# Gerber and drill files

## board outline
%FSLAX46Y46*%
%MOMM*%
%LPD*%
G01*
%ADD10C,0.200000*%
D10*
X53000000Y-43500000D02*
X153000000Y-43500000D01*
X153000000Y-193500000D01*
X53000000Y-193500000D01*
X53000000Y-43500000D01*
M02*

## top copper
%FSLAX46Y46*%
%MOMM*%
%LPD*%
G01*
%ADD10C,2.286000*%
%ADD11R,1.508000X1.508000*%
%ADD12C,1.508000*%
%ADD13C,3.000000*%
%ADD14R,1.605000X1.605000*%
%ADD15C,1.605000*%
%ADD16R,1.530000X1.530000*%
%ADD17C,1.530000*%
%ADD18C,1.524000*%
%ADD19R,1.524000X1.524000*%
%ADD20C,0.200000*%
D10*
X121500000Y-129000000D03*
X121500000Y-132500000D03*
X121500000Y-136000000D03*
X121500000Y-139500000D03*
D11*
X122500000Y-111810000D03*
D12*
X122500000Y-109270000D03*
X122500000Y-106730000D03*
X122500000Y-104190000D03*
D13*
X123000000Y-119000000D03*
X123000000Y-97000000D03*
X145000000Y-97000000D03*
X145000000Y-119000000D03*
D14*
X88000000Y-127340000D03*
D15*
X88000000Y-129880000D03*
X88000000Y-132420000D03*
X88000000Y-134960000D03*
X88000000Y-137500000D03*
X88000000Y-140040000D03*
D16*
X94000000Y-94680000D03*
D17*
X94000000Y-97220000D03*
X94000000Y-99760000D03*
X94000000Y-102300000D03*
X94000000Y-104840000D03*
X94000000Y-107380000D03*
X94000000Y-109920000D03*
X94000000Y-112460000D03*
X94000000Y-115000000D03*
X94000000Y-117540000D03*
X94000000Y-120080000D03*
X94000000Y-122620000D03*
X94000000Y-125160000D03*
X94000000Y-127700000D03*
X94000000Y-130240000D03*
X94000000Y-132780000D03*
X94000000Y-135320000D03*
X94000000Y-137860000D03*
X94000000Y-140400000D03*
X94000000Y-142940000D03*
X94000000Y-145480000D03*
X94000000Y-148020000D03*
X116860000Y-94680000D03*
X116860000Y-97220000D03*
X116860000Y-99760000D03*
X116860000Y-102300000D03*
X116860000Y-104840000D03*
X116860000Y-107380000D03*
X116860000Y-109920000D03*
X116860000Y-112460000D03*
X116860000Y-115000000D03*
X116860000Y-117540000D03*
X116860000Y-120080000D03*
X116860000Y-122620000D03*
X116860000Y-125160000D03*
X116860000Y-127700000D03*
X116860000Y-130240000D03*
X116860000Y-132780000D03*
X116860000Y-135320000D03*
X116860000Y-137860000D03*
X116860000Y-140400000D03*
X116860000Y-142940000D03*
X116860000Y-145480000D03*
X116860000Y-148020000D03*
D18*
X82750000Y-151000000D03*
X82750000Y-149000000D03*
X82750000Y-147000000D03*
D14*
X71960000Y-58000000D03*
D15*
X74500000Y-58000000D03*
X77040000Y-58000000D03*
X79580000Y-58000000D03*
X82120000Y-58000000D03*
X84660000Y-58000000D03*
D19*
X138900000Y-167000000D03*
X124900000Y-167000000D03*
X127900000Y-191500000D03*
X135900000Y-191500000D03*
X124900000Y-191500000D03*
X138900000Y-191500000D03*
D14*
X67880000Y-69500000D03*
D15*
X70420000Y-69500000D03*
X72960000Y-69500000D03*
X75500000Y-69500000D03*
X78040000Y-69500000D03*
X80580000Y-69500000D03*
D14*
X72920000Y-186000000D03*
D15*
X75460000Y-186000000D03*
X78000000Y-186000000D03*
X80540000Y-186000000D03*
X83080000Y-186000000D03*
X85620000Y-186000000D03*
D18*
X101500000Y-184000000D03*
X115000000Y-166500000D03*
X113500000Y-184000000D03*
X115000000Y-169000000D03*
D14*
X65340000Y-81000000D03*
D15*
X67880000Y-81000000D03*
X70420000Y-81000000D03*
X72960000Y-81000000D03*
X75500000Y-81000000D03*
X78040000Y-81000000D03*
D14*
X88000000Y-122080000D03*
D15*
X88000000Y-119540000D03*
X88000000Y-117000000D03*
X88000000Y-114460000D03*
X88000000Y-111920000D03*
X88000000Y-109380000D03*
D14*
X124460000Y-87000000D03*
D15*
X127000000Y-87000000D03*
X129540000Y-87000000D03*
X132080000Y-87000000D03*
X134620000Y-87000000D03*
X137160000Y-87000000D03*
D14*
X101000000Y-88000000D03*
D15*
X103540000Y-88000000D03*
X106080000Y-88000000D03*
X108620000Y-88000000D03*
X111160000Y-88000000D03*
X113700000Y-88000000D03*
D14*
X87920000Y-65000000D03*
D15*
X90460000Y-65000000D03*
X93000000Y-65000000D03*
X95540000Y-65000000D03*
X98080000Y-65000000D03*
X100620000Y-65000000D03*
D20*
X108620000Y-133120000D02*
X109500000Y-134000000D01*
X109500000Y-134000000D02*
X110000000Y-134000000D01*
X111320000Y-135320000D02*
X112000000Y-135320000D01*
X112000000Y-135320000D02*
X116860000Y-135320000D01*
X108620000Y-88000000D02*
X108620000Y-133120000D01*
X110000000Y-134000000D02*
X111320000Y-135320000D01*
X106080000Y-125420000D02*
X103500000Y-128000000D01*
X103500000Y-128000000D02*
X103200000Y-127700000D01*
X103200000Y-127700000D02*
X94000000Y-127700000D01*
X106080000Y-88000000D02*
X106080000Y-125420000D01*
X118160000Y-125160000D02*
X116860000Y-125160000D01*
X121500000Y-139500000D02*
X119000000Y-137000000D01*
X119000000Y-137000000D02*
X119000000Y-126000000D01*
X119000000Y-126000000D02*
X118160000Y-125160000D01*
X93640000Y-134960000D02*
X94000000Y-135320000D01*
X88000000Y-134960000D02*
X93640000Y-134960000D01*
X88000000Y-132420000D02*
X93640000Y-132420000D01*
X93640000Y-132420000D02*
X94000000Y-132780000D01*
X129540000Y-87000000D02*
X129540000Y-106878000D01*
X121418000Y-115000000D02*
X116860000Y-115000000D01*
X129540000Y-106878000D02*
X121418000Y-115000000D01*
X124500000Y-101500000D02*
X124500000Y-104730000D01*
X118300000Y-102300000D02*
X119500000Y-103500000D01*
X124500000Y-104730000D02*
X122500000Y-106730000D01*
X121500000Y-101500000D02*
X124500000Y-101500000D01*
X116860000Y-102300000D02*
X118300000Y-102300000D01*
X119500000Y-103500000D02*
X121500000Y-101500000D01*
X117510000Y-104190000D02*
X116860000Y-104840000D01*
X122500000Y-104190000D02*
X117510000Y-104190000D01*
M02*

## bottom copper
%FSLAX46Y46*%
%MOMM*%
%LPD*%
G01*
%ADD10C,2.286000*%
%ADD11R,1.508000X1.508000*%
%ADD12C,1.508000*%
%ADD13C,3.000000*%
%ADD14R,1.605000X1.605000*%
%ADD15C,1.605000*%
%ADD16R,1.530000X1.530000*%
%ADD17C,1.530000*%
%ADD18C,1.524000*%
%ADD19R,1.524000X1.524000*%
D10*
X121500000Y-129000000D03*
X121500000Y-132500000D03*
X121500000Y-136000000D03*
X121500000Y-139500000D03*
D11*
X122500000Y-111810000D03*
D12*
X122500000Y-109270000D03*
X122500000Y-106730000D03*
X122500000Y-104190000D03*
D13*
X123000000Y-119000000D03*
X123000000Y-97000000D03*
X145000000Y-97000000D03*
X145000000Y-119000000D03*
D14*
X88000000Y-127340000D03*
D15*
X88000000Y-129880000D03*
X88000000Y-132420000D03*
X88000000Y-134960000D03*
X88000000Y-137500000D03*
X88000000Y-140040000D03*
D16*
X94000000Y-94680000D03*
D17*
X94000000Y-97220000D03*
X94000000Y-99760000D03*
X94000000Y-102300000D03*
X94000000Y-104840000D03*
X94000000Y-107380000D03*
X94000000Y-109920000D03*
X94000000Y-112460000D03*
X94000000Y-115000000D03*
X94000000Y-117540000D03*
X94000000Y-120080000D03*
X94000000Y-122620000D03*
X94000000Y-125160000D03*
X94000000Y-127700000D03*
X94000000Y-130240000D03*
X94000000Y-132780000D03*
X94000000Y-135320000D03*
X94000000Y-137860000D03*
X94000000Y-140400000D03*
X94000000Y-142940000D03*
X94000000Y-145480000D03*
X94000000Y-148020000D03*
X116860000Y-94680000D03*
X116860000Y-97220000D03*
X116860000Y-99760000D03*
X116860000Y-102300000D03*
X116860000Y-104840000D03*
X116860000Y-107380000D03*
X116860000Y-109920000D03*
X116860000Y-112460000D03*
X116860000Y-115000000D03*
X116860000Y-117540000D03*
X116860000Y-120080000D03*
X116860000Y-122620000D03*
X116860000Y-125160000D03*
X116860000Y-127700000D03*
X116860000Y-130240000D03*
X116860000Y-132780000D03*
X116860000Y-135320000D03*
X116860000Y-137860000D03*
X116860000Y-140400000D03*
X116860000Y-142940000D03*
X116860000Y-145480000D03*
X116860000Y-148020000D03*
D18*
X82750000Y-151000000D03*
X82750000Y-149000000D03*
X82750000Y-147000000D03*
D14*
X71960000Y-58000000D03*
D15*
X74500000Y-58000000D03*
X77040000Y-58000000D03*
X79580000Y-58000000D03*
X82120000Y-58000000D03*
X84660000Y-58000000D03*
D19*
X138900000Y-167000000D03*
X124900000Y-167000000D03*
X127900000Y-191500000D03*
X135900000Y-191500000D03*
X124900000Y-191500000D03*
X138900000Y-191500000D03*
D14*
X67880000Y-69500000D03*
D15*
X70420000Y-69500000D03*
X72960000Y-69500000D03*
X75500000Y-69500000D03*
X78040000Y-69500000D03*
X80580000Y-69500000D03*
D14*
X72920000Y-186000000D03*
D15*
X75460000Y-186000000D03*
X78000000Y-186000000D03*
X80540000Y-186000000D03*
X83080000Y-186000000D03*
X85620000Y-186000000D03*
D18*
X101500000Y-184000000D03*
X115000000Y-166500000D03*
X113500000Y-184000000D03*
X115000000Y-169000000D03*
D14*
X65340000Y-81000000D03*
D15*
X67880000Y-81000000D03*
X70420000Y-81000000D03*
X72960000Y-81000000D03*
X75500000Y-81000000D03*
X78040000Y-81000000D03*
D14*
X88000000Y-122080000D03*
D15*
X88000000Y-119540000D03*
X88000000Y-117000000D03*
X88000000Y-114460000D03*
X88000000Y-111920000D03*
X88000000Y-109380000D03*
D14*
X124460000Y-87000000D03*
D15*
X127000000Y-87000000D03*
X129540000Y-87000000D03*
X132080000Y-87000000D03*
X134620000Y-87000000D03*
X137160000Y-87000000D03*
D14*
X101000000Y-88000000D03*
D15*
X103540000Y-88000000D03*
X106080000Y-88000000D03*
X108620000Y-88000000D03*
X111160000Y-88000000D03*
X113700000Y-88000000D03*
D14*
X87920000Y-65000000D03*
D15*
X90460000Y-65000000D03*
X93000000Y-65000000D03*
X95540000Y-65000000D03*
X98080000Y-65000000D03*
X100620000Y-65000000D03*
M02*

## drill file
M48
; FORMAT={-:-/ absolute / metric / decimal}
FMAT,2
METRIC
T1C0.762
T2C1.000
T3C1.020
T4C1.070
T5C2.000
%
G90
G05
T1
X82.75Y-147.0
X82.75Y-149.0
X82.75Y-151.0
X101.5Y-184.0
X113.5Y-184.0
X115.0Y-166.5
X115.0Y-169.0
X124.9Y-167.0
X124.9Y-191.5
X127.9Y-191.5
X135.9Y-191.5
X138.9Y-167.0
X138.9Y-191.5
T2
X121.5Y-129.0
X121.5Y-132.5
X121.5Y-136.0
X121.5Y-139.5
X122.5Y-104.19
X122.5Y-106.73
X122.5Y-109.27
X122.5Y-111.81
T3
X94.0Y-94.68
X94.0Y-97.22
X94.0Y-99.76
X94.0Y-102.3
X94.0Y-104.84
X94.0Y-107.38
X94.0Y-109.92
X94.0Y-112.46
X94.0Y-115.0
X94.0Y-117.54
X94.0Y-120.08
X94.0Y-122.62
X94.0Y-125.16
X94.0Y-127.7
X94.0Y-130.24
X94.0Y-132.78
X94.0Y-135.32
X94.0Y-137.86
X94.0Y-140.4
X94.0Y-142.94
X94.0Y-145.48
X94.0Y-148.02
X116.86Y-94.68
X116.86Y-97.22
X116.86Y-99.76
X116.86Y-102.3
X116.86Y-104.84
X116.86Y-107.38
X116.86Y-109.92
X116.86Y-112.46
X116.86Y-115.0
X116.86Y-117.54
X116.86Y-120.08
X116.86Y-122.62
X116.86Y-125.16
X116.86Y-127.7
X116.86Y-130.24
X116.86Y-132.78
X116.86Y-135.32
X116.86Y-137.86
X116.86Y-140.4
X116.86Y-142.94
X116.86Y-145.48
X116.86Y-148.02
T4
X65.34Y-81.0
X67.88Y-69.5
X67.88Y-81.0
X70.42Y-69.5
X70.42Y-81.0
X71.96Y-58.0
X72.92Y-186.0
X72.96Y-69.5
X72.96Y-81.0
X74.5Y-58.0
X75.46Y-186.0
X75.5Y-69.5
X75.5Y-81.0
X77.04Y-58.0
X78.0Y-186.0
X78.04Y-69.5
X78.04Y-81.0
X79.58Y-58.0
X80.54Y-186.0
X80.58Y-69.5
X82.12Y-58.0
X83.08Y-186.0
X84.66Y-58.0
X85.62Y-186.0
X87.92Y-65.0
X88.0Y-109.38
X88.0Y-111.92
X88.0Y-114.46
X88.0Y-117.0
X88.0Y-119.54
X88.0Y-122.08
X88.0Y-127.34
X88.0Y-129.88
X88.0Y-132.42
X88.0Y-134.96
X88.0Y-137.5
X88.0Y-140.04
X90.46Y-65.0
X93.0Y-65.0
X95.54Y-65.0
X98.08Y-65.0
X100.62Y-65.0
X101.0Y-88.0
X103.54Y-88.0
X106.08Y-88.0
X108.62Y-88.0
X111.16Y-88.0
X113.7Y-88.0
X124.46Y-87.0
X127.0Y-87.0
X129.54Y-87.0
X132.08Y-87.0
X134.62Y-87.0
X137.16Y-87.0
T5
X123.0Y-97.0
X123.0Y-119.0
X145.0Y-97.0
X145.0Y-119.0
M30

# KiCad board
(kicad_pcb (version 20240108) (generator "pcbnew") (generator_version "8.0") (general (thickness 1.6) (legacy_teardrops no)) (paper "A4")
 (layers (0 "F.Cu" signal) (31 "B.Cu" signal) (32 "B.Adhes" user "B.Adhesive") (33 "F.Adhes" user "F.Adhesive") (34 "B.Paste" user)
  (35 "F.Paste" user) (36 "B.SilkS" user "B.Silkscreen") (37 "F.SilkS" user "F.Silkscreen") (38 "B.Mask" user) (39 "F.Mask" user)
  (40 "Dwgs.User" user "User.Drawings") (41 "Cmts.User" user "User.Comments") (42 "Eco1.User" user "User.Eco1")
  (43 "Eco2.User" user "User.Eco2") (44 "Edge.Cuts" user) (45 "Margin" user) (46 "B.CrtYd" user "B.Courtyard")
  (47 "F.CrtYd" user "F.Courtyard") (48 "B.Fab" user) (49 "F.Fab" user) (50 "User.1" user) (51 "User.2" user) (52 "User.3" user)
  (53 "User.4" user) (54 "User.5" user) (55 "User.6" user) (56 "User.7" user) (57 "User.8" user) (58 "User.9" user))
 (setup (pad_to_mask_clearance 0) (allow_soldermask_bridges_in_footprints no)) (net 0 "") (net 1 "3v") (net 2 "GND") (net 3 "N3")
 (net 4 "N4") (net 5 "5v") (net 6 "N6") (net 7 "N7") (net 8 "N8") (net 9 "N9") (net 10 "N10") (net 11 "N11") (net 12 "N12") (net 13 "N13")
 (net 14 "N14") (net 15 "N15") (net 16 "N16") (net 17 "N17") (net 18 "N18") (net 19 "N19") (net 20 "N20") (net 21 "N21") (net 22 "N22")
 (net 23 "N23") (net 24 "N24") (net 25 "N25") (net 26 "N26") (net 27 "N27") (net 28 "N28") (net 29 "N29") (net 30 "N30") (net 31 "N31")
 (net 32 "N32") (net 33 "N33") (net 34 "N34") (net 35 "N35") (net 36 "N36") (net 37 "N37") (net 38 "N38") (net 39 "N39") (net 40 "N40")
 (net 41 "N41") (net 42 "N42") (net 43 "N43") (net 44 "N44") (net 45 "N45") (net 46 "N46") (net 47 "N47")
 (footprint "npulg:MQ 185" (layer "F.Cu") (at 144 132.5 -90)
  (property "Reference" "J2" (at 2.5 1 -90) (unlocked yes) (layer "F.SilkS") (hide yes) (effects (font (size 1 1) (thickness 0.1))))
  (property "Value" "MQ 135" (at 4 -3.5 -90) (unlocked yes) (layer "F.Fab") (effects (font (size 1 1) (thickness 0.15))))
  (pad "1" thru_hole circle (at -3.5 22.5 270) (size 2.286 2.286) (drill 1) (layers "*.Cu" "*.Mask") (remove_unused_layers no) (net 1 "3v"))
  (pad "2" thru_hole circle (at 0 22.5 270) (size 2.286 2.286) (drill 1) (layers "*.Cu" "*.Mask") (remove_unused_layers no) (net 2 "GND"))
  (pad "3" thru_hole circle (at 3.5 22.5 270) (size 2.286 2.286) (drill 1) (layers "*.Cu" "*.Mask") (remove_unused_layers no) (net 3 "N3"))
  (pad "4" thru_hole circle (at 7 22.5 270) (size 2.286 2.286) (drill 1) (layers "*.Cu" "*.Mask") (remove_unused_layers no) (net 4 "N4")))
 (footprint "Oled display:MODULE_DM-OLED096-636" (layer "F.Cu") (at 134 108 90)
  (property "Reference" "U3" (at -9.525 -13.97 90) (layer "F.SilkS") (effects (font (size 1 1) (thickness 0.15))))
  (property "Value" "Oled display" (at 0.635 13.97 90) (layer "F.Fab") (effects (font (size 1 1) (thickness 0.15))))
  (pad "1" thru_hole rect (at -3.81 -11.5 90) (size 1.508 1.508) (drill 1) (layers "*.Cu" "*.Mask") (remove_unused_layers no) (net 2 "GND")
   (solder_mask_margin 0.102))
  (pad "2" thru_hole circle (at -1.27 -11.5 90) (size 1.508 1.508) (drill 1) (layers "*.Cu" "*.Mask") (remove_unused_layers no) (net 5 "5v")
   (solder_mask_margin 0.102))
  (pad "3" thru_hole circle (at 1.27 -11.5 90) (size 1.508 1.508) (drill 1) (layers "*.Cu" "*.Mask") (remove_unused_layers no) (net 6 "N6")
   (solder_mask_margin 0.102))
  (pad "4" thru_hole circle (at 3.81 -11.5 90) (size 1.508 1.508) (drill 1) (layers "*.Cu" "*.Mask") (remove_unused_layers no) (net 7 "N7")
   (solder_mask_margin 0.102))
  (pad "S1" thru_hole circle (at -11 -11 90) (size 3 3) (drill 2) (layers "*.Cu" "*.Mask") (remove_unused_layers no)
   (solder_mask_margin 0.102))
  (pad "S2" thru_hole circle (at 11 -11 90) (size 3 3) (drill 2) (layers "*.Cu" "*.Mask") (remove_unused_layers no)
   (solder_mask_margin 0.102))
  (pad "S3" thru_hole circle (at 11 11 90) (size 3 3) (drill 2) (layers "*.Cu" "*.Mask") (remove_unused_layers no)
   (solder_mask_margin 0.102))
  (pad "S4" thru_hole circle (at -11 11 90) (size 3 3) (drill 2) (layers "*.Cu" "*.Mask") (remove_unused_layers no)
   (solder_mask_margin 0.102)))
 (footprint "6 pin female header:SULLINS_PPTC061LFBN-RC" (layer "F.Cu") (at 88 133.69 -90)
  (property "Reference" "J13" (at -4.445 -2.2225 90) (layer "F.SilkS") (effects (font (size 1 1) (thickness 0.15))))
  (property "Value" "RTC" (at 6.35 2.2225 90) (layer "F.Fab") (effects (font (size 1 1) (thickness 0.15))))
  (pad "1" thru_hole rect (at -6.35 0 270) (size 1.605 1.605) (drill 1.07) (layers "*.Cu" "*.Mask") (remove_unused_layers no) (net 5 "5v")
   (solder_mask_margin 0.102))
  (pad "2" thru_hole circle (at -3.81 0 270) (size 1.605 1.605) (drill 1.07) (layers "*.Cu" "*.Mask") (remove_unused_layers no)
   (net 2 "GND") (solder_mask_margin 0.102))
  (pad "3" thru_hole circle (at -1.27 0 270) (size 1.605 1.605) (drill 1.07) (layers "*.Cu" "*.Mask") (remove_unused_layers no) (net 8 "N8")
   (solder_mask_margin 0.102))
  (pad "4" thru_hole circle (at 1.27 0 270) (size 1.605 1.605) (drill 1.07) (layers "*.Cu" "*.Mask") (remove_unused_layers no) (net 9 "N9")
   (solder_mask_margin 0.102))
  (pad "5" thru_hole circle (at 3.81 0 270) (size 1.605 1.605) (drill 1.07) (layers "*.Cu" "*.Mask") (remove_unused_layers no)
   (solder_mask_margin 0.102))
  (pad "6" thru_hole circle (at 6.35 0 270) (size 1.605 1.605) (drill 1.07) (layers "*.Cu" "*.Mask") (remove_unused_layers no)
   (solder_mask_margin 0.102)))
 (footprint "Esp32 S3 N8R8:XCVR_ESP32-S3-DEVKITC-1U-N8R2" (layer "F.Cu") (at 105.43 124.65)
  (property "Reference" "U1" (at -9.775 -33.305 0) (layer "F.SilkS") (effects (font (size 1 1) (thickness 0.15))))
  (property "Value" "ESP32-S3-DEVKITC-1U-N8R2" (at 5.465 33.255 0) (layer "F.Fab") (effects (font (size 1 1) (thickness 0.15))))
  (pad "J1_1" thru_hole rect (at -11.43 -29.97) (size 1.53 1.53) (drill 1.02) (layers "*.Cu" "*.Mask") (remove_unused_layers no)
   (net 1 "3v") (solder_mask_margin 0.102))
  (pad "J1_2" thru_hole circle (at -11.43 -27.43) (size 1.53 1.53) (drill 1.02) (layers "*.Cu" "*.Mask") (remove_unused_layers no)
   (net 1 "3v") (solder_mask_margin 0.102))
  (pad "J1_3" thru_hole circle (at -11.43 -24.89) (size 1.53 1.53) (drill 1.02) (layers "*.Cu" "*.Mask") (remove_unused_layers no)
   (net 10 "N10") (solder_mask_margin 0.102))
  (pad "J1_4" thru_hole circle (at -11.43 -22.35) (size 1.53 1.53) (drill 1.02) (layers "*.Cu" "*.Mask") (remove_unused_layers no)
   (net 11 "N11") (solder_mask_margin 0.102))
  (pad "J1_5" thru_hole circle (at -11.43 -19.81) (size 1.53 1.53) (drill 1.02) (layers "*.Cu" "*.Mask") (remove_unused_layers no)
   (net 5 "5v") (solder_mask_margin 0.102))
  (pad "J1_6" thru_hole circle (at -11.43 -17.27) (size 1.53 1.53) (drill 1.02) (layers "*.Cu" "*.Mask") (remove_unused_layers no)
   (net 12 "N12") (solder_mask_margin 0.102))
  (pad "J1_7" thru_hole circle (at -11.43 -14.73) (size 1.53 1.53) (drill 1.02) (layers "*.Cu" "*.Mask") (remove_unused_layers no)
   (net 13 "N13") (solder_mask_margin 0.102))
  (pad "J1_8" thru_hole circle (at -11.43 -12.19) (size 1.53 1.53) (drill 1.02) (layers "*.Cu" "*.Mask") (remove_unused_layers no)
   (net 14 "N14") (solder_mask_margin 0.102))
  (pad "J1_9" thru_hole circle (at -11.43 -9.65) (size 1.53 1.53) (drill 1.02) (layers "*.Cu" "*.Mask") (remove_unused_layers no)
   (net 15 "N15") (solder_mask_margin 0.102))
  (pad "J1_10" thru_hole circle (at -11.43 -7.11) (size 1.53 1.53) (drill 1.02) (layers "*.Cu" "*.Mask") (remove_unused_layers no)
   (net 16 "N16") (solder_mask_margin 0.102))
  (pad "J1_11" thru_hole circle (at -11.43 -4.57) (size 1.53 1.53) (drill 1.02) (layers "*.Cu" "*.Mask") (remove_unused_layers no)
   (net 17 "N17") (solder_mask_margin 0.102))
  (pad "J1_12" thru_hole circle (at -11.43 -2.03) (size 1.53 1.53) (drill 1.02) (layers "*.Cu" "*.Mask") (remove_unused_layers no)
   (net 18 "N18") (solder_mask_margin 0.102))
  (pad "J1_13" thru_hole circle (at -11.43 0.51) (size 1.53 1.53) (drill 1.02) (layers "*.Cu" "*.Mask") (remove_unused_layers no)
   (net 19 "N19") (solder_mask_margin 0.102))
  (pad "J1_14" thru_hole circle (at -11.43 3.05) (size 1.53 1.53) (drill 1.02) (layers "*.Cu" "*.Mask") (remove_unused_layers no)
   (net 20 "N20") (solder_mask_margin 0.102))
  (pad "J1_15" thru_hole circle (at -11.43 5.59) (size 1.53 1.53) (drill 1.02) (layers "*.Cu" "*.Mask") (remove_unused_layers no)
   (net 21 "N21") (solder_mask_margin 0.102))
  (pad "J1_16" thru_hole circle (at -11.43 8.13) (size 1.53 1.53) (drill 1.02) (layers "*.Cu" "*.Mask") (remove_unused_layers no)
   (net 8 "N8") (solder_mask_margin 0.102))
  (pad "J1_17" thru_hole circle (at -11.43 10.67) (size 1.53 1.53) (drill 1.02) (layers "*.Cu" "*.Mask") (remove_unused_layers no)
   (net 9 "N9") (solder_mask_margin 0.102))
  (pad "J1_18" thru_hole circle (at -11.43 13.21) (size 1.53 1.53) (drill 1.02) (layers "*.Cu" "*.Mask") (remove_unused_layers no)
   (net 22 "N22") (solder_mask_margin 0.102))
  (pad "J1_19" thru_hole circle (at -11.43 15.75) (size 1.53 1.53) (drill 1.02) (layers "*.Cu" "*.Mask") (remove_unused_layers no)
   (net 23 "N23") (solder_mask_margin 0.102))
  (pad "J1_20" thru_hole circle (at -11.43 18.29) (size 1.53 1.53) (drill 1.02) (layers "*.Cu" "*.Mask") (remove_unused_layers no)
   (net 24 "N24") (solder_mask_margin 0.102))
  (pad "J1_21" thru_hole circle (at -11.43 20.83) (size 1.53 1.53) (drill 1.02) (layers "*.Cu" "*.Mask") (remove_unused_layers no)
   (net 5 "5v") (solder_mask_margin 0.102))
  (pad "J1_22" thru_hole circle (at -11.43 23.37) (size 1.53 1.53) (drill 1.02) (layers "*.Cu" "*.Mask") (remove_unused_layers no)
   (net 2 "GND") (solder_mask_margin 0.102))
  (pad "J3_1" thru_hole circle (at 11.43 -29.97) (size 1.53 1.53) (drill 1.02) (layers "*.Cu" "*.Mask") (remove_unused_layers no)
   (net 2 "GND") (solder_mask_margin 0.102))
  (pad "J3_2" thru_hole circle (at 11.43 -27.43) (size 1.53 1.53) (drill 1.02) (layers "*.Cu" "*.Mask") (remove_unused_layers no)
   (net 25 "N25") (solder_mask_margin 0.102))
  (pad "J3_3" thru_hole circle (at 11.43 -24.89) (size 1.53 1.53) (drill 1.02) (layers "*.Cu" "*.Mask") (remove_unused_layers no)
   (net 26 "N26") (solder_mask_margin 0.102))
  (pad "J3_4" thru_hole circle (at 11.43 -22.35) (size 1.53 1.53) (drill 1.02) (layers "*.Cu" "*.Mask") (remove_unused_layers no)
   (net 6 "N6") (solder_mask_margin 0.102))
  (pad "J3_5" thru_hole circle (at 11.43 -19.81) (size 1.53 1.53) (drill 1.02) (layers "*.Cu" "*.Mask") (remove_unused_layers no)
   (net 7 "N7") (solder_mask_margin 0.102))
  (pad "J3_6" thru_hole circle (at 11.43 -17.27) (size 1.53 1.53) (drill 1.02) (layers "*.Cu" "*.Mask") (remove_unused_layers no)
   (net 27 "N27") (solder_mask_margin 0.102))
  (pad "J3_7" thru_hole circle (at 11.43 -14.73) (size 1.53 1.53) (drill 1.02) (layers "*.Cu" "*.Mask") (remove_unused_layers no)
   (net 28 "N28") (solder_mask_margin 0.102))
  (pad "J3_8" thru_hole circle (at 11.43 -12.19) (size 1.53 1.53) (drill 1.02) (layers "*.Cu" "*.Mask") (remove_unused_layers no)
   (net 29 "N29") (solder_mask_margin 0.102))
  (pad "J3_9" thru_hole circle (at 11.43 -9.65) (size 1.53 1.53) (drill 1.02) (layers "*.Cu" "*.Mask") (remove_unused_layers no)
   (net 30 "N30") (solder_mask_margin 0.102))
  (pad "J3_10" thru_hole circle (at 11.43 -7.11) (size 1.53 1.53) (drill 1.02) (layers "*.Cu" "*.Mask") (remove_unused_layers no)
   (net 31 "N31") (solder_mask_margin 0.102))
  (pad "J3_11" thru_hole circle (at 11.43 -4.57) (size 1.53 1.53) (drill 1.02) (layers "*.Cu" "*.Mask") (remove_unused_layers no)
   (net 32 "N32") (solder_mask_margin 0.102))
  (pad "J3_12" thru_hole circle (at 11.43 -2.03) (size 1.53 1.53) (drill 1.02) (layers "*.Cu" "*.Mask") (remove_unused_layers no)
   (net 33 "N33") (solder_mask_margin 0.102))
  (pad "J3_13" thru_hole circle (at 11.43 0.51) (size 1.53 1.53) (drill 1.02) (layers "*.Cu" "*.Mask") (remove_unused_layers no)
   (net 4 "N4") (solder_mask_margin 0.102))
  (pad "J3_14" thru_hole circle (at 11.43 3.05) (size 1.53 1.53) (drill 1.02) (layers "*.Cu" "*.Mask") (remove_unused_layers no)
   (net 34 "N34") (solder_mask_margin 0.102))
  (pad "J3_15" thru_hole circle (at 11.43 5.59) (size 1.53 1.53) (drill 1.02) (layers "*.Cu" "*.Mask") (remove_unused_layers no)
   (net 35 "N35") (solder_mask_margin 0.102))
  (pad "J3_16" thru_hole circle (at 11.43 8.13) (size 1.53 1.53) (drill 1.02) (layers "*.Cu" "*.Mask") (remove_unused_layers no)
   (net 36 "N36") (solder_mask_margin 0.102))
  (pad "J3_17" thru_hole circle (at 11.43 10.67) (size 1.53 1.53) (drill 1.02) (layers "*.Cu" "*.Mask") (remove_unused_layers no)
   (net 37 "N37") (solder_mask_margin 0.102))
  (pad "J3_18" thru_hole circle (at 11.43 13.21) (size 1.53 1.53) (drill 1.02) (layers "*.Cu" "*.Mask") (remove_unused_layers no)
   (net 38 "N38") (solder_mask_margin 0.102))
  (pad "J3_19" thru_hole circle (at 11.43 15.75) (size 1.53 1.53) (drill 1.02) (layers "*.Cu" "*.Mask") (remove_unused_layers no)
   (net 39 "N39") (solder_mask_margin 0.102))
  (pad "J3_20" thru_hole circle (at 11.43 18.29) (size 1.53 1.53) (drill 1.02) (layers "*.Cu" "*.Mask") (remove_unused_layers no)
   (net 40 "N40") (solder_mask_margin 0.102))
  (pad "J3_21" thru_hole circle (at 11.43 20.83) (size 1.53 1.53) (drill 1.02) (layers "*.Cu" "*.Mask") (remove_unused_layers no)
   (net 2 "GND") (solder_mask_margin 0.102))
  (pad "J3_22" thru_hole circle (at 11.43 23.37) (size 1.53 1.53) (drill 1.02) (layers "*.Cu" "*.Mask") (remove_unused_layers no)
   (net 2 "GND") (solder_mask_margin 0.102)))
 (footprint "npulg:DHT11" (layer "F.Cu") (at 75.25 148 90)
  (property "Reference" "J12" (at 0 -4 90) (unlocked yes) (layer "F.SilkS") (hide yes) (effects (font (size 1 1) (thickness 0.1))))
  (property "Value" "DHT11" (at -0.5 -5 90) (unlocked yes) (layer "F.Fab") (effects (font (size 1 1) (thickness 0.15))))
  (pad "1" thru_hole circle (at -3 7.5 90) (size 1.524 1.524) (drill 0.762) (layers "*.Cu" "*.Mask") (remove_unused_layers no) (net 2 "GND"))
  (pad "2" thru_hole circle (at -1 7.5 90) (size 1.524 1.524) (drill 0.762) (layers "*.Cu" "*.Mask") (remove_unused_layers no)
   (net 33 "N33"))
  (pad "3" thru_hole circle (at 1 7.5 90) (size 1.524 1.524) (drill 0.762) (layers "*.Cu" "*.Mask") (remove_unused_layers no) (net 5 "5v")))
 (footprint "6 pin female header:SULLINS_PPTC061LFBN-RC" (layer "F.Cu") (at 78.31 58)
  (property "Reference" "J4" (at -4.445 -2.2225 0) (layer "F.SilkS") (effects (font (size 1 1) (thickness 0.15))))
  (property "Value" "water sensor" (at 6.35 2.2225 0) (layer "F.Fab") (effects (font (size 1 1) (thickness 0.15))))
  (pad "1" thru_hole rect (at -6.35 0) (size 1.605 1.605) (drill 1.07) (layers "*.Cu" "*.Mask") (remove_unused_layers no) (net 5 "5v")
   (solder_mask_margin 0.102))
  (pad "2" thru_hole circle (at -3.81 0) (size 1.605 1.605) (drill 1.07) (layers "*.Cu" "*.Mask") (remove_unused_layers no) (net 2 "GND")
   (solder_mask_margin 0.102))
  (pad "3" thru_hole circle (at -1.27 0) (size 1.605 1.605) (drill 1.07) (layers "*.Cu" "*.Mask") (remove_unused_layers no) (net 11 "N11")
   (solder_mask_margin 0.102))
  (pad "4" thru_hole circle (at 1.27 0) (size 1.605 1.605) (drill 1.07) (layers "*.Cu" "*.Mask") (remove_unused_layers no)
   (solder_mask_margin 0.102))
  (pad "5" thru_hole circle (at 3.81 0) (size 1.605 1.605) (drill 1.07) (layers "*.Cu" "*.Mask") (remove_unused_layers no)
   (solder_mask_margin 0.102))
  (pad "6" thru_hole circle (at 6.35 0) (size 1.605 1.605) (drill 1.07) (layers "*.Cu" "*.Mask") (remove_unused_layers no)
   (solder_mask_margin 0.102)))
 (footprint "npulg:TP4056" (layer "F.Cu") (at 130.9 171.5)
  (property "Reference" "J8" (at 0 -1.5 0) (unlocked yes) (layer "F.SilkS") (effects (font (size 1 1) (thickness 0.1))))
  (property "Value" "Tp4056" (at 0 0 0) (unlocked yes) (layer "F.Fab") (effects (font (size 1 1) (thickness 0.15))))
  (pad "+IN" thru_hole rect (at 8 -4.5) (size 1.524 1.524) (drill 0.762) (layers "*.Cu" "*.Mask") (remove_unused_layers no))
  (pad "-IN" thru_hole rect (at -6 -4.5) (size 1.524 1.524) (drill 0.762) (layers "*.Cu" "*.Mask") (remove_unused_layers no))
  (pad "BAT+" thru_hole rect (at -3 20) (size 1.524 1.524) (drill 0.762) (layers "*.Cu" "*.Mask") (remove_unused_layers no))
  (pad "BAT-" thru_hole rect (at 5 20) (size 1.524 1.524) (drill 0.762) (layers "*.Cu" "*.Mask") (remove_unused_layers no))
  (pad "OUT+" thru_hole rect (at -6 20) (size 1.524 1.524) (drill 0.762) (layers "*.Cu" "*.Mask") (remove_unused_layers no))
  (pad "OUT-" thru_hole rect (at 8 20) (size 1.524 1.524) (drill 0.762) (layers "*.Cu" "*.Mask") (remove_unused_layers no)))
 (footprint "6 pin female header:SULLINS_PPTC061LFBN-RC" (layer "F.Cu") (at 74.23 69.5)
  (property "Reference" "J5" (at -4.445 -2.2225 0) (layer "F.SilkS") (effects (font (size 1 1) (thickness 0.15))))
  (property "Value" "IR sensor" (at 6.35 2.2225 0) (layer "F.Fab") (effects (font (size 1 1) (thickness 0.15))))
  (pad "1" thru_hole rect (at -6.35 0) (size 1.605 1.605) (drill 1.07) (layers "*.Cu" "*.Mask") (remove_unused_layers no) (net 5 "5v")
   (solder_mask_margin 0.102))
  (pad "2" thru_hole circle (at -3.81 0) (size 1.605 1.605) (drill 1.07) (layers "*.Cu" "*.Mask") (remove_unused_layers no) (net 2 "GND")
   (solder_mask_margin 0.102))
  (pad "3" thru_hole circle (at -1.27 0) (size 1.605 1.605) (drill 1.07) (layers "*.Cu" "*.Mask") (remove_unused_layers no) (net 36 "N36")
   (solder_mask_margin 0.102))
  (pad "4" thru_hole circle (at 1.27 0) (size 1.605 1.605) (drill 1.07) (layers "*.Cu" "*.Mask") (remove_unused_layers no)
   (solder_mask_margin 0.102))
  (pad "5" thru_hole circle (at 3.81 0) (size 1.605 1.605) (drill 1.07) (layers "*.Cu" "*.Mask") (remove_unused_layers no)
   (solder_mask_margin 0.102))
  (pad "6" thru_hole circle (at 6.35 0) (size 1.605 1.605) (drill 1.07) (layers "*.Cu" "*.Mask") (remove_unused_layers no)
   (solder_mask_margin 0.102)))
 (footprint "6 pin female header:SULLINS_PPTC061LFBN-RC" (layer "F.Cu") (at 79.27 186)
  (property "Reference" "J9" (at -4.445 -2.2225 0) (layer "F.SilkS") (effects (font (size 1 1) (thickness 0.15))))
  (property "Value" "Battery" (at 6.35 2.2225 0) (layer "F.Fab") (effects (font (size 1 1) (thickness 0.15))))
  (pad "1" thru_hole rect (at -6.35 0) (size 1.605 1.605) (drill 1.07) (layers "*.Cu" "*.Mask") (remove_unused_layers no) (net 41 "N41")
   (solder_mask_margin 0.102))
  (pad "2" thru_hole circle (at -3.81 0) (size 1.605 1.605) (drill 1.07) (layers "*.Cu" "*.Mask") (remove_unused_layers no) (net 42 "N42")
   (solder_mask_margin 0.102))
  (pad "3" thru_hole circle (at -1.27 0) (size 1.605 1.605) (drill 1.07) (layers "*.Cu" "*.Mask") (remove_unused_layers no)
   (solder_mask_margin 0.102))
  (pad "4" thru_hole circle (at 1.27 0) (size 1.605 1.605) (drill 1.07) (layers "*.Cu" "*.Mask") (remove_unused_layers no)
   (solder_mask_margin 0.102))
  (pad "5" thru_hole circle (at 3.81 0) (size 1.605 1.605) (drill 1.07) (layers "*.Cu" "*.Mask") (remove_unused_layers no)
   (solder_mask_margin 0.102))
  (pad "6" thru_hole circle (at 6.35 0) (size 1.605 1.605) (drill 1.07) (layers "*.Cu" "*.Mask") (remove_unused_layers no)
   (solder_mask_margin 0.102)))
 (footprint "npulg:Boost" (layer "F.Cu") (at 105.5 172)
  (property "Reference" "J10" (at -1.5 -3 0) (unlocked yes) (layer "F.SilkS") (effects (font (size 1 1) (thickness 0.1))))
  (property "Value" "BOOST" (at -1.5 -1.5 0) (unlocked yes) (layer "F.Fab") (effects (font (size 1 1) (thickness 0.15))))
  (pad "+" thru_hole circle (at -4 12) (size 1.524 1.524) (drill 0.762) (layers "*.Cu" "*.Mask") (remove_unused_layers no))
  (pad "+5v" thru_hole circle (at 9.5 -5.5) (size 1.524 1.524) (drill 0.762) (layers "*.Cu" "*.Mask") (remove_unused_layers no))
  (pad "-" thru_hole circle (at 8 12) (size 1.524 1.524) (drill 0.762) (layers "*.Cu" "*.Mask") (remove_unused_layers no))
  (pad "GND" thru_hole circle (at 9.5 -3) (size 1.524 1.524) (drill 0.762) (layers "*.Cu" "*.Mask") (remove_unused_layers no)))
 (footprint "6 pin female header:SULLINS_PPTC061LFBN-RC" (layer "F.Cu") (at 71.69 81)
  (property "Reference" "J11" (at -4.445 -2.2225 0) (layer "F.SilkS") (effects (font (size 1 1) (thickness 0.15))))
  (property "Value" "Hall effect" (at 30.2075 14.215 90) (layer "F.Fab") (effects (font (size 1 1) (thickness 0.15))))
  (pad "1" thru_hole rect (at -6.35 0) (size 1.605 1.605) (drill 1.07) (layers "*.Cu" "*.Mask") (remove_unused_layers no) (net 5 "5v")
   (solder_mask_margin 0.102))
  (pad "2" thru_hole circle (at -3.81 0) (size 1.605 1.605) (drill 1.07) (layers "*.Cu" "*.Mask") (remove_unused_layers no) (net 2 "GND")
   (solder_mask_margin 0.102))
  (pad "3" thru_hole circle (at -1.27 0) (size 1.605 1.605) (drill 1.07) (layers "*.Cu" "*.Mask") (remove_unused_layers no) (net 34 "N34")
   (solder_mask_margin 0.102))
  (pad "4" thru_hole circle (at 1.27 0) (size 1.605 1.605) (drill 1.07) (layers "*.Cu" "*.Mask") (remove_unused_layers no)
   (solder_mask_margin 0.102))
  (pad "5" thru_hole circle (at 3.81 0) (size 1.605 1.605) (drill 1.07) (layers "*.Cu" "*.Mask") (remove_unused_layers no)
   (solder_mask_margin 0.102))
  (pad "6" thru_hole circle (at 6.35 0) (size 1.605 1.605) (drill 1.07) (layers "*.Cu" "*.Mask") (remove_unused_layers no)
   (solder_mask_margin 0.102)))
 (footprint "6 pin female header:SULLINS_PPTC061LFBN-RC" (layer "F.Cu") (at 88 115.73 90)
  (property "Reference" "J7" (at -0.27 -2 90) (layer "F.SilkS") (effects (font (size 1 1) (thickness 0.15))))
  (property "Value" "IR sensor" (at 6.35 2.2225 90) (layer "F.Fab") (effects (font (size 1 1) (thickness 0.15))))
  (pad "1" thru_hole rect (at -6.35 0 90) (size 1.605 1.605) (drill 1.07) (layers "*.Cu" "*.Mask") (remove_unused_layers no) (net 5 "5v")
   (solder_mask_margin 0.102))
  (pad "2" thru_hole circle (at -3.81 0 90) (size 1.605 1.605) (drill 1.07) (layers "*.Cu" "*.Mask") (remove_unused_layers no) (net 2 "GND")
   (solder_mask_margin 0.102))
  (pad "3" thru_hole circle (at -1.27 0 90) (size 1.605 1.605) (drill 1.07) (layers "*.Cu" "*.Mask") (remove_unused_layers no)
   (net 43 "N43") (solder_mask_margin 0.102))
  (pad "4" thru_hole circle (at 1.27 0 90) (size 1.605 1.605) (drill 1.07) (layers "*.Cu" "*.Mask") (remove_unused_layers no)
   (solder_mask_margin 0.102))
  (pad "5" thru_hole circle (at 3.81 0 90) (size 1.605 1.605) (drill 1.07) (layers "*.Cu" "*.Mask") (remove_unused_layers no)
   (solder_mask_margin 0.102))
  (pad "6" thru_hole circle (at 6.35 0 90) (size 1.605 1.605) (drill 1.07) (layers "*.Cu" "*.Mask") (remove_unused_layers no)
   (solder_mask_margin 0.102)))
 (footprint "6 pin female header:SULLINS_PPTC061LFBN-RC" (layer "F.Cu") (at 130.81 87)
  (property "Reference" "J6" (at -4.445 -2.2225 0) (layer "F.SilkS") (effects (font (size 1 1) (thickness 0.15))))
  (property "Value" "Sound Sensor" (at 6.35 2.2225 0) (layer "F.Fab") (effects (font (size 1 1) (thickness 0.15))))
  (pad "1" thru_hole rect (at -6.35 0) (size 1.605 1.605) (drill 1.07) (layers "*.Cu" "*.Mask") (remove_unused_layers no) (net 5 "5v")
   (solder_mask_margin 0.102))
  (pad "2" thru_hole circle (at -3.81 0) (size 1.605 1.605) (drill 1.07) (layers "*.Cu" "*.Mask") (remove_unused_layers no) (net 2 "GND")
   (solder_mask_margin 0.102))
  (pad "3" thru_hole circle (at -1.27 0) (size 1.605 1.605) (drill 1.07) (layers "*.Cu" "*.Mask") (remove_unused_layers no) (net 30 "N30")
   (solder_mask_margin 0.102))
  (pad "4" thru_hole circle (at 1.27 0) (size 1.605 1.605) (drill 1.07) (layers "*.Cu" "*.Mask") (remove_unused_layers no) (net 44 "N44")
   (solder_mask_margin 0.102))
  (pad "5" thru_hole circle (at 3.81 0) (size 1.605 1.605) (drill 1.07) (layers "*.Cu" "*.Mask") (remove_unused_layers no)
   (solder_mask_margin 0.102))
  (pad "6" thru_hole circle (at 6.35 0) (size 1.605 1.605) (drill 1.07) (layers "*.Cu" "*.Mask") (remove_unused_layers no)
   (solder_mask_margin 0.102)))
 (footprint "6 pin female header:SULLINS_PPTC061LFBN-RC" (layer "F.Cu") (at 107.35 88)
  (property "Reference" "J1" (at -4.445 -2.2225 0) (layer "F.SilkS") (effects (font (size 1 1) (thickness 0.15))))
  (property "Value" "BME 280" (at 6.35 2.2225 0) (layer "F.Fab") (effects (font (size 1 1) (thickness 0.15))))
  (pad "1" thru_hole rect (at -6.35 0) (size 1.605 1.605) (drill 1.07) (layers "*.Cu" "*.Mask") (remove_unused_layers no) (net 1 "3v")
   (solder_mask_margin 0.102))
  (pad "2" thru_hole circle (at -3.81 0) (size 1.605 1.605) (drill 1.07) (layers "*.Cu" "*.Mask") (remove_unused_layers no) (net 2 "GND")
   (solder_mask_margin 0.102))
  (pad "3" thru_hole circle (at -1.27 0) (size 1.605 1.605) (drill 1.07) (layers "*.Cu" "*.Mask") (remove_unused_layers no) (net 20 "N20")
   (solder_mask_margin 0.102))
  (pad "4" thru_hole circle (at 1.27 0) (size 1.605 1.605) (drill 1.07) (layers "*.Cu" "*.Mask") (remove_unused_layers no) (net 37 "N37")
   (solder_mask_margin 0.102))
  (pad "5" thru_hole circle (at 3.81 0) (size 1.605 1.605) (drill 1.07) (layers "*.Cu" "*.Mask") (remove_unused_layers no) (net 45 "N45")
   (solder_mask_margin 0.102))
  (pad "6" thru_hole circle (at 6.35 0) (size 1.605 1.605) (drill 1.07) (layers "*.Cu" "*.Mask") (remove_unused_layers no) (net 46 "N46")
   (solder_mask_margin 0.102)))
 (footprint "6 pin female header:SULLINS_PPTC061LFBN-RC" (layer "F.Cu") (at 94.27 65)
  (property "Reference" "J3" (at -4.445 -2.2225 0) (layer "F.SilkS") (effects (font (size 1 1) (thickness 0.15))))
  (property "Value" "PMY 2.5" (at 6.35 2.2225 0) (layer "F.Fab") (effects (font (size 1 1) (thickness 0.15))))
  (pad "1" thru_hole rect (at -6.35 0) (size 1.605 1.605) (drill 1.07) (layers "*.Cu" "*.Mask") (remove_unused_layers no) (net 5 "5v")
   (solder_mask_margin 0.102))
  (pad "2" thru_hole circle (at -3.81 0) (size 1.605 1.605) (drill 1.07) (layers "*.Cu" "*.Mask") (remove_unused_layers no) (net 5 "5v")
   (solder_mask_margin 0.102))
  (pad "3" thru_hole circle (at -1.27 0) (size 1.605 1.605) (drill 1.07) (layers "*.Cu" "*.Mask") (remove_unused_layers no) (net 2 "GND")
   (solder_mask_margin 0.102))
  (pad "4" thru_hole circle (at 1.27 0) (size 1.605 1.605) (drill 1.07) (layers "*.Cu" "*.Mask") (remove_unused_layers no) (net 17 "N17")
   (solder_mask_margin 0.102))
  (pad "5" thru_hole circle (at 3.81 0) (size 1.605 1.605) (drill 1.07) (layers "*.Cu" "*.Mask") (remove_unused_layers no) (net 2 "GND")
   (solder_mask_margin 0.102))
  (pad "6" thru_hole circle (at 6.35 0) (size 1.605 1.605) (drill 1.07) (layers "*.Cu" "*.Mask") (remove_unused_layers no) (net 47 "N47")
   (solder_mask_margin 0.102)))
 (gr_rect (start 53 43.5) (end 153 193.5) (stroke (width 0.2) (type default)) (fill none) (layer "Edge.Cuts"))
 (segment (start 108.62 133.12) (end 109.5 134) (width 0.2) (layer "F.Cu") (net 37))
 (segment (start 109.5 134) (end 110 134) (width 0.2) (layer "F.Cu") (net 37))
 (segment (start 111.32 135.32) (end 112 135.32) (width 0.2) (layer "F.Cu") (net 37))
 (segment (start 112 135.32) (end 116.86 135.32) (width 0.2) (layer "F.Cu") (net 37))
 (segment (start 108.62 88) (end 108.62 133.12) (width 0.2) (layer "F.Cu") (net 37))
 (segment (start 110 134) (end 111.32 135.32) (width 0.2) (layer "F.Cu") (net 37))
 (segment (start 106.08 125.42) (end 103.5 128) (width 0.2) (layer "F.Cu") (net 20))
 (segment (start 103.5 128) (end 103.2 127.7) (width 0.2) (layer "F.Cu") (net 20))
 (segment (start 103.2 127.7) (end 94 127.7) (width 0.2) (layer "F.Cu") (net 20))
 (segment (start 106.08 88) (end 106.08 125.42) (width 0.2) (layer "F.Cu") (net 20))
 (segment (start 118.16 125.16) (end 116.86 125.16) (width 0.2) (layer "F.Cu") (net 4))
 (segment (start 121.5 139.5) (end 119 137) (width 0.2) (layer "F.Cu") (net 4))
 (segment (start 119 137) (end 119 126) (width 0.2) (layer "F.Cu") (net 4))
 (segment (start 119 126) (end 118.16 125.16) (width 0.2) (layer "F.Cu") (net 4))
 (segment (start 93.64 134.96) (end 94 135.32) (width 0.2) (layer "F.Cu") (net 9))
 (segment (start 88 134.96) (end 93.64 134.96) (width 0.2) (layer "F.Cu") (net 9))
 (segment (start 88 132.42) (end 93.64 132.42) (width 0.2) (layer "F.Cu") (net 8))
 (segment (start 93.64 132.42) (end 94 132.78) (width 0.2) (layer "F.Cu") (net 8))
 (segment (start 129.54 87) (end 129.54 106.878) (width 0.2) (layer "F.Cu") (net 30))
 (segment (start 121.418 115) (end 116.86 115) (width 0.2) (layer "F.Cu") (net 30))
 (segment (start 129.54 106.878) (end 121.418 115) (width 0.2) (layer "F.Cu") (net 30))
 (segment (start 124.5 101.5) (end 124.5 104.73) (width 0.2) (layer "F.Cu") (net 6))
 (segment (start 118.3 102.3) (end 119.5 103.5) (width 0.2) (layer "F.Cu") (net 6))
 (segment (start 124.5 104.73) (end 122.5 106.73) (width 0.2) (layer "F.Cu") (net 6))
 (segment (start 121.5 101.5) (end 124.5 101.5) (width 0.2) (layer "F.Cu") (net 6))
 (segment (start 116.86 102.3) (end 118.3 102.3) (width 0.2) (layer "F.Cu") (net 6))
 (segment (start 119.5 103.5) (end 121.5 101.5) (width 0.2) (layer "F.Cu") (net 6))
 (segment (start 117.51 104.19) (end 116.86 104.84) (width 0.2) (layer "F.Cu") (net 7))
 (segment (start 122.5 104.19) (end 117.51 104.19) (width 0.2) (layer "F.Cu") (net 7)))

